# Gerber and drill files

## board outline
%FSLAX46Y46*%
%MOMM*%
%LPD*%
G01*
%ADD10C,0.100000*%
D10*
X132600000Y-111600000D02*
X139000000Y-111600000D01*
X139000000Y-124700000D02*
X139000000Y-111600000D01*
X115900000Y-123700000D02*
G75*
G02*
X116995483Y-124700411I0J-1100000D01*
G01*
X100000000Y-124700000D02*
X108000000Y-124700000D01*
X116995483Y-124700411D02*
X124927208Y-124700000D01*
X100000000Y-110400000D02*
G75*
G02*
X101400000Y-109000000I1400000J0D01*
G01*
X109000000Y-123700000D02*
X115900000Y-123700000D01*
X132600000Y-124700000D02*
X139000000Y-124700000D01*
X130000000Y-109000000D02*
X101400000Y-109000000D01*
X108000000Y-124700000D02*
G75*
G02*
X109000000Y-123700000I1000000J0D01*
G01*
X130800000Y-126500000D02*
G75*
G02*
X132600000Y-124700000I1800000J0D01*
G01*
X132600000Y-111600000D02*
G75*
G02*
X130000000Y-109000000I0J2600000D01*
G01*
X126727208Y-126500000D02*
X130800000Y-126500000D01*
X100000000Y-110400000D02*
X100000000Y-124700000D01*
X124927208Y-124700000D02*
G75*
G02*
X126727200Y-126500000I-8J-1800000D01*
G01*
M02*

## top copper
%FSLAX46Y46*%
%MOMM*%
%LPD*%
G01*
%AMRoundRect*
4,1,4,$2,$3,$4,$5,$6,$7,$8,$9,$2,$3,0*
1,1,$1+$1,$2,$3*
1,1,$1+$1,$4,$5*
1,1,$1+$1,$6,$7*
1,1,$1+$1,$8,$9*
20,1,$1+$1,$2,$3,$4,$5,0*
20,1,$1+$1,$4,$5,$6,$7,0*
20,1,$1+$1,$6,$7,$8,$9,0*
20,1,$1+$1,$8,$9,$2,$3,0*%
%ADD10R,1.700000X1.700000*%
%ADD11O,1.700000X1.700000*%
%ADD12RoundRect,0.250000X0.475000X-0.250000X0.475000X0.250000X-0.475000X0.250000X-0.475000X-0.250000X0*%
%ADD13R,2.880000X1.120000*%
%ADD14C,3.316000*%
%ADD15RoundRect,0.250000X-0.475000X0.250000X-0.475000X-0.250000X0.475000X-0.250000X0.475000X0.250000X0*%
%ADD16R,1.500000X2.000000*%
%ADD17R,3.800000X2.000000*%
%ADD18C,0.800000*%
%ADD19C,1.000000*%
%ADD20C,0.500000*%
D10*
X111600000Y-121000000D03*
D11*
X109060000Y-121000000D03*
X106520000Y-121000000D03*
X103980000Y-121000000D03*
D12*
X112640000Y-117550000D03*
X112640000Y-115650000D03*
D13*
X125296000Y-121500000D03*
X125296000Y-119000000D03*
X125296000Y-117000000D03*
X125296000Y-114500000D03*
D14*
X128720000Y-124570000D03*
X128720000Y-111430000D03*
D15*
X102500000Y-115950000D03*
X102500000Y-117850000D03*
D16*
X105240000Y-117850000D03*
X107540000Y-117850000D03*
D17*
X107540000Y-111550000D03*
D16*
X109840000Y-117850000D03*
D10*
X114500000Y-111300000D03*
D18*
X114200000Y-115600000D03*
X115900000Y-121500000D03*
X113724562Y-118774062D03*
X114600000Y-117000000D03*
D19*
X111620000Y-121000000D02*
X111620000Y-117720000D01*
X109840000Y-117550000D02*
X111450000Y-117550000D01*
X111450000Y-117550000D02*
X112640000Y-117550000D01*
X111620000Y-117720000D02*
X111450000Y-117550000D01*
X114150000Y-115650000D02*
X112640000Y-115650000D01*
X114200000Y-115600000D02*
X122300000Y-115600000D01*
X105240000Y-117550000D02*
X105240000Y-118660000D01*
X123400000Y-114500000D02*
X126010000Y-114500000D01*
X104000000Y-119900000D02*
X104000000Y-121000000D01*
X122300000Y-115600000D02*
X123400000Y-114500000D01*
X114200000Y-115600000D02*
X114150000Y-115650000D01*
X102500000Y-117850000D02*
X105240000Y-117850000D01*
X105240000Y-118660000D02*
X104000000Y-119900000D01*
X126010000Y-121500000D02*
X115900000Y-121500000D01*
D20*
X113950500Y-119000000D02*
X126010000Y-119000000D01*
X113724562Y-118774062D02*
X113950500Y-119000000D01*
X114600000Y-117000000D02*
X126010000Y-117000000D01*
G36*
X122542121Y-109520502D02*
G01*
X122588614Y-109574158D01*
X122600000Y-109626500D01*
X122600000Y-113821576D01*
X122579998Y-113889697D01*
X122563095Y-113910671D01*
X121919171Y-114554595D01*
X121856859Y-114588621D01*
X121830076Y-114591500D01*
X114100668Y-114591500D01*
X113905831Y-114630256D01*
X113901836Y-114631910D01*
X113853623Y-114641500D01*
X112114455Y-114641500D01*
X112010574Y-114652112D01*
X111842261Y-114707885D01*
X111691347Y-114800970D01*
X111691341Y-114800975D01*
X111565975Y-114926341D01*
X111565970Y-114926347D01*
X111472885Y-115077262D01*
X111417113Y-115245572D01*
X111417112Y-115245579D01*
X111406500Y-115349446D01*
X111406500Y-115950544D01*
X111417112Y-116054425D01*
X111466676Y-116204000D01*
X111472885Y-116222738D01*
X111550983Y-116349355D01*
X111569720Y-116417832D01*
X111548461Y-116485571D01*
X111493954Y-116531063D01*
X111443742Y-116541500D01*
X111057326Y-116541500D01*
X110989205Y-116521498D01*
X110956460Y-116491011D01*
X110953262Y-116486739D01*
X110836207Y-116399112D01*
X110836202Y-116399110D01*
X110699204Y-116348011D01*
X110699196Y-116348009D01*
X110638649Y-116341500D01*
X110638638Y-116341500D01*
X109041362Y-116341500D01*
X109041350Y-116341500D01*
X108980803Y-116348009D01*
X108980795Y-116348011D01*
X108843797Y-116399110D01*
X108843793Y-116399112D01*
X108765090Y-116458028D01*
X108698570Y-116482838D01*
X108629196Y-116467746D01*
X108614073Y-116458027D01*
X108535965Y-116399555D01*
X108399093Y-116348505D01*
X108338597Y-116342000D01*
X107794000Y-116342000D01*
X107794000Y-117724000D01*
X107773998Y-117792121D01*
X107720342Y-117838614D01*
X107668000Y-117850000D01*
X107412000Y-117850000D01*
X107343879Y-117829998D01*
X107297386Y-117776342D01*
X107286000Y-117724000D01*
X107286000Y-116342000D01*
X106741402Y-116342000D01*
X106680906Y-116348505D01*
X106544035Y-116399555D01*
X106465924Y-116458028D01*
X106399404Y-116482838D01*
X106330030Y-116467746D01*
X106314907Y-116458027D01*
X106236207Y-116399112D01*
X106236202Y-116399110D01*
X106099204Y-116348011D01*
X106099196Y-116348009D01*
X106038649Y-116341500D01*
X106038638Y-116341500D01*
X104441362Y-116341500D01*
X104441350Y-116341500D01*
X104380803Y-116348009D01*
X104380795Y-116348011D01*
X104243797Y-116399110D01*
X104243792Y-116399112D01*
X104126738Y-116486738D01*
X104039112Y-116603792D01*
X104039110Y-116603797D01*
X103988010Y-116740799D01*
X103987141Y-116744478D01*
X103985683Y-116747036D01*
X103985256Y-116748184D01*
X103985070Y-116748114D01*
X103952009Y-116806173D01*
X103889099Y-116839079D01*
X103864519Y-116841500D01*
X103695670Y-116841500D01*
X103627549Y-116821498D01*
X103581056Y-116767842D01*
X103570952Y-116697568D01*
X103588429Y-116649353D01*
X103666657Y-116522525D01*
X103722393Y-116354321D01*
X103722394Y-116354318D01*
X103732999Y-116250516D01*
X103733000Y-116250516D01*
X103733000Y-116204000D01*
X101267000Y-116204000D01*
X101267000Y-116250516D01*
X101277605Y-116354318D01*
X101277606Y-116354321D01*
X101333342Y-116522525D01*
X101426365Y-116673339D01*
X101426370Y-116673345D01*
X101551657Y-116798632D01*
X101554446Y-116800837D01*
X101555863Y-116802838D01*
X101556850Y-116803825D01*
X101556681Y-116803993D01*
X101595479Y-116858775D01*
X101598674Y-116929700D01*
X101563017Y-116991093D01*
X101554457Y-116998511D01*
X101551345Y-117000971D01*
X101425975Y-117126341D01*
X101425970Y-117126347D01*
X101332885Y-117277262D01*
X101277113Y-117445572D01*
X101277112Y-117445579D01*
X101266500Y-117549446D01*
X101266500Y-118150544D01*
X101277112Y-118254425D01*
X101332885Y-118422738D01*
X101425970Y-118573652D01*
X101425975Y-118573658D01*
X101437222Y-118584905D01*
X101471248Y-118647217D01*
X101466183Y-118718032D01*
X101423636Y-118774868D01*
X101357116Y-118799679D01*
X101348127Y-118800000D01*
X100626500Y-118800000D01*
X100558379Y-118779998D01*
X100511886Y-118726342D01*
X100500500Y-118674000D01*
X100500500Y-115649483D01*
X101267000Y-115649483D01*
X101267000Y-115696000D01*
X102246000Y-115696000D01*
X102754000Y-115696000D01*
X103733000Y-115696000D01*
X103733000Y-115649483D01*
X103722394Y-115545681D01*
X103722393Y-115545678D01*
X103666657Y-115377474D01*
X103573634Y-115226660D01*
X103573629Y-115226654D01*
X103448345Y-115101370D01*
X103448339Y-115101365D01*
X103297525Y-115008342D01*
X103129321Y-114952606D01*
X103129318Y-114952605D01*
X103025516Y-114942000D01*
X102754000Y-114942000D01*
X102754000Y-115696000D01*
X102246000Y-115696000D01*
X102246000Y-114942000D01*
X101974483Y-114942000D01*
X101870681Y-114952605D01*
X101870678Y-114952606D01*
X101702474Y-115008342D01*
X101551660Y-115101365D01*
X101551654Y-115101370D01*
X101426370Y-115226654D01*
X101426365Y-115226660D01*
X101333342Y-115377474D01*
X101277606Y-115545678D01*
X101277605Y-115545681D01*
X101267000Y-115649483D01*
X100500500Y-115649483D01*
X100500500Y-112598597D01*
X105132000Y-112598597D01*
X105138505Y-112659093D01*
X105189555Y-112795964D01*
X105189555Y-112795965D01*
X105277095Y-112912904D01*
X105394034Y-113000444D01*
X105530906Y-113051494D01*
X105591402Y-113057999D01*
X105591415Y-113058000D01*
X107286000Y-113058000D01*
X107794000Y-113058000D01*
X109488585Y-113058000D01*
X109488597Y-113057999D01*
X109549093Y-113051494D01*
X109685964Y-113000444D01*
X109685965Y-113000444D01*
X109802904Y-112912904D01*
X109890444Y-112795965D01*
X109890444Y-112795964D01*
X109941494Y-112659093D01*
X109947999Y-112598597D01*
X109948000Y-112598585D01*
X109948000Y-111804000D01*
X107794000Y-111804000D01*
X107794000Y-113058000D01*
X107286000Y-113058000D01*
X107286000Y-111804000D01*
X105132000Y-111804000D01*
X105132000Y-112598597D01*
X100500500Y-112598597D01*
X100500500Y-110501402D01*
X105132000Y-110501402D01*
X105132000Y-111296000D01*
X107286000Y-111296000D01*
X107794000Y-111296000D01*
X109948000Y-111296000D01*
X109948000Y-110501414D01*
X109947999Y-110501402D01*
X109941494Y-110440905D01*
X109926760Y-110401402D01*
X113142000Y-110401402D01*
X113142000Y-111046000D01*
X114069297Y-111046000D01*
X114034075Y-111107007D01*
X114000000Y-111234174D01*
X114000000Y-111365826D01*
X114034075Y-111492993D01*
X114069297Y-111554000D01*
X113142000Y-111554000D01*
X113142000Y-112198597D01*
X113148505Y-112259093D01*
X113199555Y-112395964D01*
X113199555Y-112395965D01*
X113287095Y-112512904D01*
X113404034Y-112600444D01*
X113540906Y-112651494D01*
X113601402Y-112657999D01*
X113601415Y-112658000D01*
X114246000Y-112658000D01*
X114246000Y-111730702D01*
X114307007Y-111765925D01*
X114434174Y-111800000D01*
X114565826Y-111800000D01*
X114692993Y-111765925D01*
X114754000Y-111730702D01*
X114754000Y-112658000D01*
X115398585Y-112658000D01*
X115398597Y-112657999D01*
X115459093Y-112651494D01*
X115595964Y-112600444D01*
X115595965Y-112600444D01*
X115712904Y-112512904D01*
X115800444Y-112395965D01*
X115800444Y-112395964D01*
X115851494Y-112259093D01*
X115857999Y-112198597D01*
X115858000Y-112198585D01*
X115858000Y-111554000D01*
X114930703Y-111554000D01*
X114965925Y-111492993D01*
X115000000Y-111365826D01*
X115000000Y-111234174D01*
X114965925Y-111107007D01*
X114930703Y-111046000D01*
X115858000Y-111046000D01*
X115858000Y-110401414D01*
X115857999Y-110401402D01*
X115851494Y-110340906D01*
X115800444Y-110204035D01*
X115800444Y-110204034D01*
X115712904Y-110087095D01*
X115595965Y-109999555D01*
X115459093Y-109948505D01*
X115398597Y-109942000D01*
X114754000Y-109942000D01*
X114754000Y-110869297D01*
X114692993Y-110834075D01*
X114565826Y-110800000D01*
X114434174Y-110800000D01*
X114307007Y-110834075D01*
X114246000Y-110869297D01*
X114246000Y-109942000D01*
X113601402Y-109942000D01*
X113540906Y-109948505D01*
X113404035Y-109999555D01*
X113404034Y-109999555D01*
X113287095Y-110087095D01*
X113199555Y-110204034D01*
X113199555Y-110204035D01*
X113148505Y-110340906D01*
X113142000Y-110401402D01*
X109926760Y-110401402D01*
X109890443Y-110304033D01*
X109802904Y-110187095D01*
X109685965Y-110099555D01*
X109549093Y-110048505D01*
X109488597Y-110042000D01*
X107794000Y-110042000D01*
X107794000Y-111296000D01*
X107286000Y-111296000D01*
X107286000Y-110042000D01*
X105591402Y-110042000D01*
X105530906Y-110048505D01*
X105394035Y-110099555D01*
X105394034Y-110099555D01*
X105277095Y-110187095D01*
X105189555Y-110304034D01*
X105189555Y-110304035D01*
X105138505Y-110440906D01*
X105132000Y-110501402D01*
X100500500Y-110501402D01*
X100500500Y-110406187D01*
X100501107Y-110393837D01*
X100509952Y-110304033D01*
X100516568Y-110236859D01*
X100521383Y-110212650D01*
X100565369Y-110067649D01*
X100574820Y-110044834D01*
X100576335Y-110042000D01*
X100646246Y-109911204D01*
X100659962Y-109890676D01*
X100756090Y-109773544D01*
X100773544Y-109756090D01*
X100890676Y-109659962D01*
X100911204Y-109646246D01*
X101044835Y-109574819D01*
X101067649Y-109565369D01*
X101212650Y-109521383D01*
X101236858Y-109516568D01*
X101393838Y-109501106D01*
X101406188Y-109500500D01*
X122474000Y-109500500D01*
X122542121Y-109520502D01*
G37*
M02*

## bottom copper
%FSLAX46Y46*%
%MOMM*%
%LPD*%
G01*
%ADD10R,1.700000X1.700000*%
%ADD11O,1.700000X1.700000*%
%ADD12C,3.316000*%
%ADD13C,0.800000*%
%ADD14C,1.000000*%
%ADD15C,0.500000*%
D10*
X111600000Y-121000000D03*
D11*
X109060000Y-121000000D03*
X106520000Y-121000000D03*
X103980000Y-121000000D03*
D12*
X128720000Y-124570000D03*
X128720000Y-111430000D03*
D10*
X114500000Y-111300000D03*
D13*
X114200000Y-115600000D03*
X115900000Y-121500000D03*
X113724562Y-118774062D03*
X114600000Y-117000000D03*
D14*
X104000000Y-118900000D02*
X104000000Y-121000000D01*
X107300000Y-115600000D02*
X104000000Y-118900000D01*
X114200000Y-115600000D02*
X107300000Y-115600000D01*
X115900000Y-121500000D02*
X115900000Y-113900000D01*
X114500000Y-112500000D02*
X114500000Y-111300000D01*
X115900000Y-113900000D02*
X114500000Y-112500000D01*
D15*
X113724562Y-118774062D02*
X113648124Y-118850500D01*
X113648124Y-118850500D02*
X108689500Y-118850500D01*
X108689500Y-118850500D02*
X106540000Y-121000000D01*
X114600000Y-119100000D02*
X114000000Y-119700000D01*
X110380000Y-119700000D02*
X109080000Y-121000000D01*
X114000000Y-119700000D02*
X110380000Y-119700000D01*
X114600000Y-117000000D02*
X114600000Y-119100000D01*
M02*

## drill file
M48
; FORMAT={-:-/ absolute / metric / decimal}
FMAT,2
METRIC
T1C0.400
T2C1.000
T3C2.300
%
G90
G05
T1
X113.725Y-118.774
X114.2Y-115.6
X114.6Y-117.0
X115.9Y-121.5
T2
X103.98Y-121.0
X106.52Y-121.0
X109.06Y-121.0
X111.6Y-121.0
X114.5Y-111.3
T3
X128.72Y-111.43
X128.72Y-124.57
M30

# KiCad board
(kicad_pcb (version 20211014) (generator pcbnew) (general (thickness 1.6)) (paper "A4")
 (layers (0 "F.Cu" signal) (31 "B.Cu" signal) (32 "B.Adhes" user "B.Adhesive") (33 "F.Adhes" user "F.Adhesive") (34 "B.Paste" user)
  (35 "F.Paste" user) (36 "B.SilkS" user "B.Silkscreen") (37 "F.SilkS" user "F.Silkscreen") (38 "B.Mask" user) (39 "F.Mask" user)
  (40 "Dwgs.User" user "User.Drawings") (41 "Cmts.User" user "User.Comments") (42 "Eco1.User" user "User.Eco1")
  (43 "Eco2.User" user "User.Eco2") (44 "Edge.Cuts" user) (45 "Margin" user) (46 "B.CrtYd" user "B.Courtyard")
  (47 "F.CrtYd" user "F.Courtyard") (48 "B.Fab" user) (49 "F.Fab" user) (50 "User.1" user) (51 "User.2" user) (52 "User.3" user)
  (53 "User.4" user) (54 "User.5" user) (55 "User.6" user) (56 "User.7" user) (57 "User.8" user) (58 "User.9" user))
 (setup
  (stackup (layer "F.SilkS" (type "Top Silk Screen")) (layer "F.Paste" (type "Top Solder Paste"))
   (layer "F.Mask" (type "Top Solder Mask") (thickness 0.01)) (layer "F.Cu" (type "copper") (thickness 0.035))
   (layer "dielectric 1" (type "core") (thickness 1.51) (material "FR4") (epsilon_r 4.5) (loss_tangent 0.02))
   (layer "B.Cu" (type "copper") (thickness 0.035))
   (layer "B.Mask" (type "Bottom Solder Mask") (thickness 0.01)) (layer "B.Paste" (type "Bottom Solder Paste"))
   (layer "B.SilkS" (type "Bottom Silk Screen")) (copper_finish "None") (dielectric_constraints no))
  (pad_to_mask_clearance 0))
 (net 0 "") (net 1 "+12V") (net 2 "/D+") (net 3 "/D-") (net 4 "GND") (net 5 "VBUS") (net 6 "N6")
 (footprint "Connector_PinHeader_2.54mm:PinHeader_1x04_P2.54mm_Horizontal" (layer "F.Cu") (at 111.6 121 -90)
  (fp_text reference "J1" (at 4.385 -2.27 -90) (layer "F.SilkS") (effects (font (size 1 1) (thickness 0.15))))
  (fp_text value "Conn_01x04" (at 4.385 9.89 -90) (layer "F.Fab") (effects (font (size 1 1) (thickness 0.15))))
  (pad "1" thru_hole rect (at 0 0 270) (size 1.7 1.7) (drill 1) (layers *.Cu *.Mask) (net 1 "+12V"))
  (pad "2" thru_hole oval (at 0 2.54 270) (size 1.7 1.7) (drill 1) (layers *.Cu *.Mask) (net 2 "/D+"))
  (pad "3" thru_hole oval (at 0 5.08 270) (size 1.7 1.7) (drill 1) (layers *.Cu *.Mask) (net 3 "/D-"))
  (pad "4" thru_hole oval (at 0 7.62 270) (size 1.7 1.7) (drill 1) (layers *.Cu *.Mask) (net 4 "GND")))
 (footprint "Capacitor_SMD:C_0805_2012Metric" (layer "F.Cu") (at 112.64 116.6 90)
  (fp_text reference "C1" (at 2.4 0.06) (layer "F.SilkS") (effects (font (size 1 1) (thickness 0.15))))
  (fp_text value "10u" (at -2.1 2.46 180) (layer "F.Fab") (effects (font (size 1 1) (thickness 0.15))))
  (pad "1" smd roundrect (at -0.95 0 90) (size 1 1.45) (layers "F.Cu" "F.Paste" "F.Mask") (roundrect_rratio 0.25) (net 1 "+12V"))
  (pad "2" smd roundrect (at 0.95 0 90) (size 1 1.45) (layers "F.Cu" "F.Paste" "F.Mask") (roundrect_rratio 0.25) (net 4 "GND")))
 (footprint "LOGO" (layer "F.Cu") (at 121 111.5)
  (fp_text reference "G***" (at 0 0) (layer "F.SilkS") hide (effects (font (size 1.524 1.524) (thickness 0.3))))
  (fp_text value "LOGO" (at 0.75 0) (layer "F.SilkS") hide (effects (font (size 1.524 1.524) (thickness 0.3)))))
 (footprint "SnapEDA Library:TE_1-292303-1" (layer "F.Cu") (at 132 118 90)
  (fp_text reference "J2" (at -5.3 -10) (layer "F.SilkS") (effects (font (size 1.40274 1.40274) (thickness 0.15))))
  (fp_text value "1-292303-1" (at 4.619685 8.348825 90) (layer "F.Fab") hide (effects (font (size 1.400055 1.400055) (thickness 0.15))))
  (pad "1" smd rect (at -3.5 -5.99 90) (size 1.12 2.88) (drill (offset 0 -0.714)) (layers "F.Cu" "F.Paste" "F.Mask") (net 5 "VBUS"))
  (pad "2" smd rect (at -1 -5.99 90) (size 1.12 2.88) (drill (offset 0 -0.714)) (layers "F.Cu" "F.Paste" "F.Mask") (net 3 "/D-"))
  (pad "3" smd rect (at 1 -5.99 90) (size 1.12 2.88) (drill (offset 0 -0.714)) (layers "F.Cu" "F.Paste" "F.Mask") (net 2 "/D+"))
  (pad "4" smd rect (at 3.5 -5.99 90) (size 1.12 2.88) (drill (offset 0 -0.714)) (layers "F.Cu" "F.Paste" "F.Mask") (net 4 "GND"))
  (pad "S1" thru_hole circle (at -6.57 -3.28 90) (size 3.316 3.316) (drill 2.3) (layers *.Cu *.Mask) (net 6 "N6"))
  (pad "S2" thru_hole circle (at 6.57 -3.28 90) (size 3.316 3.316) (drill 2.3) (layers *.Cu *.Mask) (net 6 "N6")))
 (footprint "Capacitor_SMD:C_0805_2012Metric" (layer "F.Cu") (at 102.5 116.9 -90)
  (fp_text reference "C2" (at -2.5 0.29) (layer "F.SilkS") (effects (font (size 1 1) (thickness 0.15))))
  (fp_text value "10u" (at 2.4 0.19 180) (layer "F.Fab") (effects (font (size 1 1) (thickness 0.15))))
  (pad "1" smd roundrect (at -0.95 0 270) (size 1 1.45) (layers "F.Cu" "F.Paste" "F.Mask") (roundrect_rratio 0.25) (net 5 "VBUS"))
  (pad "2" smd roundrect locked (at 0.95 0 270) (size 1 1.45) (layers "F.Cu" "F.Paste" "F.Mask") (roundrect_rratio 0.25) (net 4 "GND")))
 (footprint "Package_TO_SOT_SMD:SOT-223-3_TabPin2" (layer "F.Cu") (at 107.54 114.7 90)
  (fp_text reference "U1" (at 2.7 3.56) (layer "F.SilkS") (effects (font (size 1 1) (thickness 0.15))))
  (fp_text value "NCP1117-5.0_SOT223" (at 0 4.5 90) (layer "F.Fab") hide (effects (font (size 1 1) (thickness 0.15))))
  (pad "1" smd rect (at -3.15 -2.3 90) (size 2 1.5) (layers "F.Cu" "F.Paste" "F.Mask") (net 4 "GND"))
  (pad "2" smd rect (at -3.15 0 90) (size 2 1.5) (layers "F.Cu" "F.Paste" "F.Mask") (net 5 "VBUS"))
  (pad "2" smd rect (at 3.15 0 90) (size 2 3.8) (layers "F.Cu" "F.Paste" "F.Mask") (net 5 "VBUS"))
  (pad "3" smd rect (at -3.15 2.3 90) (size 2 1.5) (layers "F.Cu" "F.Paste" "F.Mask") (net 1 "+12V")))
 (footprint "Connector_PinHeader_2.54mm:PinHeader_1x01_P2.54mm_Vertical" (layer "F.Cu") (at 114.5 111.3)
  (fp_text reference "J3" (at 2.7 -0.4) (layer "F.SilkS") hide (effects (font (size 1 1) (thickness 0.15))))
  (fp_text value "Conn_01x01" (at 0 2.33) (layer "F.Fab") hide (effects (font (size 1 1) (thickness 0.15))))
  (pad "1" thru_hole rect (at 0 0) (size 1.7 1.7) (drill 1) (layers *.Cu *.Mask) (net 5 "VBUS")))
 (gr_line (start 132.6 111.6) (end 139 111.6) (layer "Edge.Cuts") (width 0.1))
 (gr_line (start 139 124.7) (end 139 111.6) (layer "Edge.Cuts") (width 0.1))
 (gr_arc (start 115.9 123.7) (mid 116.641772 123.987735) (end 116.995483 124.700411) (layer "Edge.Cuts") (width 0.1))
 (gr_line (start 100 124.7) (end 108 124.7) (layer "Edge.Cuts") (width 0.1))
 (gr_line (start 116.995483 124.700411) (end 124.927208 124.7) (layer "Edge.Cuts") (width 0.1))
 (gr_arc (start 100 110.4) (mid 100.410051 109.410051) (end 101.4 109) (layer "Edge.Cuts") (width 0.1))
 (gr_line (start 109 123.7) (end 115.9 123.7) (layer "Edge.Cuts") (width 0.1))
 (gr_line (start 132.6 124.7) (end 139 124.7) (layer "Edge.Cuts") (width 0.1))
 (gr_line (start 130 109) (end 101.4 109) (layer "Edge.Cuts") (width 0.1))
 (gr_arc (start 108 124.7) (mid 108.292893 123.992893) (end 109 123.7) (layer "Edge.Cuts") (width 0.1))
 (gr_arc (start 130.8 126.5) (mid 131.327208 125.227208) (end 132.6 124.7) (layer "Edge.Cuts") (width 0.1))
 (gr_arc (start 132.6 111.6) (mid 130.761522 110.838478) (end 130 109) (layer "Edge.Cuts") (width 0.1))
 (gr_line (start 126.727208 126.5) (end 130.8 126.5) (layer "Edge.Cuts") (width 0.1))
 (gr_line (start 100 110.4) (end 100 124.7) (layer "Edge.Cuts") (width 0.1))
 (gr_arc (start 124.927208 124.7) (mid 126.2 125.227208) (end 126.727208 126.5) (layer "Edge.Cuts") (width 0.1))
 (segment (start 111.62 121) (end 111.62 117.72) (width 1) (layer "F.Cu") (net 1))
 (segment (start 109.84 117.55) (end 111.45 117.55) (width 1) (layer "F.Cu") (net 1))
 (segment (start 111.45 117.55) (end 112.64 117.55) (width 1) (layer "F.Cu") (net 1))
 (segment (start 111.62 117.72) (end 111.45 117.55) (width 1) (layer "F.Cu") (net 1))
 (segment (start 114.15 115.65) (end 112.64 115.65) (width 1) (layer "F.Cu") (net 4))
 (segment (start 114.2 115.6) (end 122.3 115.6) (width 1) (layer "F.Cu") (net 4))
 (segment (start 105.24 117.55) (end 105.24 118.66) (width 1) (layer "F.Cu") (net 4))
 (segment (start 123.4 114.5) (end 126.01 114.5) (width 1) (layer "F.Cu") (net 4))
 (segment (start 104 119.9) (end 104 121) (width 1) (layer "F.Cu") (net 4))
 (segment (start 122.3 115.6) (end 123.4 114.5) (width 1) (layer "F.Cu") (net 4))
 (segment (start 114.2 115.6) (end 114.15 115.65) (width 1) (layer "F.Cu") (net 4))
 (segment (start 102.5 117.85) (end 105.24 117.85) (width 1) (layer "F.Cu") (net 4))
 (segment (start 105.24 118.66) (end 104 119.9) (width 1) (layer "F.Cu") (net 4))
 (via (at 114.2 115.6) (size 0.8) (drill 0.4) (layers "F.Cu" "B.Cu") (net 4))
 (segment (start 104 118.9) (end 104 121) (width 1) (layer "B.Cu") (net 4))
 (segment (start 107.3 115.6) (end 104 118.9) (width 1) (layer "B.Cu") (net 4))
 (segment (start 114.2 115.6) (end 107.3 115.6) (width 1) (layer "B.Cu") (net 4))
 (segment (start 126.01 121.5) (end 115.9 121.5) (width 1) (layer "F.Cu") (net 5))
 (via (at 115.9 121.5) (size 0.8) (drill 0.4) (layers "F.Cu" "B.Cu") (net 5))
 (segment (start 115.9 121.5) (end 115.9 113.9) (width 1) (layer "B.Cu") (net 5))
 (segment (start 114.5 112.5) (end 114.5 111.3) (width 1) (layer "B.Cu") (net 5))
 (segment (start 115.9 113.9) (end 114.5 112.5) (width 1) (layer "B.Cu") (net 5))
 (segment (start 113.9505 119) (end 126.01 119) (width 0.5) (layer "F.Cu") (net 3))
 (segment (start 113.724562 118.774062) (end 113.9505 119) (width 0.5) (layer "F.Cu") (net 3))
 (via (at 113.724562 118.774062) (size 0.8) (drill 0.4) (layers "F.Cu" "B.Cu") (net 3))
 (segment (start 113.724562 118.774062) (end 113.648124 118.8505) (width 0.5) (layer "B.Cu") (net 3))
 (segment (start 113.648124 118.8505) (end 108.6895 118.8505) (width 0.5) (layer "B.Cu") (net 3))
 (segment (start 108.6895 118.8505) (end 106.54 121) (width 0.5) (layer "B.Cu") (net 3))
 (segment (start 114.6 117) (end 126.01 117) (width 0.5) (layer "F.Cu") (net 2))
 (via (at 114.6 117) (size 0.8) (drill 0.4) (layers "F.Cu" "B.Cu") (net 2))
 (segment (start 114.6 119.1) (end 114 119.7) (width 0.5) (layer "B.Cu") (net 2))
 (segment (start 110.38 119.7) (end 109.08 121) (width 0.5) (layer "B.Cu") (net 2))
 (segment (start 114 119.7) (end 110.38 119.7) (width 0.5) (layer "B.Cu") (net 2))
 (segment (start 114.6 117) (end 114.6 119.1) (width 0.5) (layer "B.Cu") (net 2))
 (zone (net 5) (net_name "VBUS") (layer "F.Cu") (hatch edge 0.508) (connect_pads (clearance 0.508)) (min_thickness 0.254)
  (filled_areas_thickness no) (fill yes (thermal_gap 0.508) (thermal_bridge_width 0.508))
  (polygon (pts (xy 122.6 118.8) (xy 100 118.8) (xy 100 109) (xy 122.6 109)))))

